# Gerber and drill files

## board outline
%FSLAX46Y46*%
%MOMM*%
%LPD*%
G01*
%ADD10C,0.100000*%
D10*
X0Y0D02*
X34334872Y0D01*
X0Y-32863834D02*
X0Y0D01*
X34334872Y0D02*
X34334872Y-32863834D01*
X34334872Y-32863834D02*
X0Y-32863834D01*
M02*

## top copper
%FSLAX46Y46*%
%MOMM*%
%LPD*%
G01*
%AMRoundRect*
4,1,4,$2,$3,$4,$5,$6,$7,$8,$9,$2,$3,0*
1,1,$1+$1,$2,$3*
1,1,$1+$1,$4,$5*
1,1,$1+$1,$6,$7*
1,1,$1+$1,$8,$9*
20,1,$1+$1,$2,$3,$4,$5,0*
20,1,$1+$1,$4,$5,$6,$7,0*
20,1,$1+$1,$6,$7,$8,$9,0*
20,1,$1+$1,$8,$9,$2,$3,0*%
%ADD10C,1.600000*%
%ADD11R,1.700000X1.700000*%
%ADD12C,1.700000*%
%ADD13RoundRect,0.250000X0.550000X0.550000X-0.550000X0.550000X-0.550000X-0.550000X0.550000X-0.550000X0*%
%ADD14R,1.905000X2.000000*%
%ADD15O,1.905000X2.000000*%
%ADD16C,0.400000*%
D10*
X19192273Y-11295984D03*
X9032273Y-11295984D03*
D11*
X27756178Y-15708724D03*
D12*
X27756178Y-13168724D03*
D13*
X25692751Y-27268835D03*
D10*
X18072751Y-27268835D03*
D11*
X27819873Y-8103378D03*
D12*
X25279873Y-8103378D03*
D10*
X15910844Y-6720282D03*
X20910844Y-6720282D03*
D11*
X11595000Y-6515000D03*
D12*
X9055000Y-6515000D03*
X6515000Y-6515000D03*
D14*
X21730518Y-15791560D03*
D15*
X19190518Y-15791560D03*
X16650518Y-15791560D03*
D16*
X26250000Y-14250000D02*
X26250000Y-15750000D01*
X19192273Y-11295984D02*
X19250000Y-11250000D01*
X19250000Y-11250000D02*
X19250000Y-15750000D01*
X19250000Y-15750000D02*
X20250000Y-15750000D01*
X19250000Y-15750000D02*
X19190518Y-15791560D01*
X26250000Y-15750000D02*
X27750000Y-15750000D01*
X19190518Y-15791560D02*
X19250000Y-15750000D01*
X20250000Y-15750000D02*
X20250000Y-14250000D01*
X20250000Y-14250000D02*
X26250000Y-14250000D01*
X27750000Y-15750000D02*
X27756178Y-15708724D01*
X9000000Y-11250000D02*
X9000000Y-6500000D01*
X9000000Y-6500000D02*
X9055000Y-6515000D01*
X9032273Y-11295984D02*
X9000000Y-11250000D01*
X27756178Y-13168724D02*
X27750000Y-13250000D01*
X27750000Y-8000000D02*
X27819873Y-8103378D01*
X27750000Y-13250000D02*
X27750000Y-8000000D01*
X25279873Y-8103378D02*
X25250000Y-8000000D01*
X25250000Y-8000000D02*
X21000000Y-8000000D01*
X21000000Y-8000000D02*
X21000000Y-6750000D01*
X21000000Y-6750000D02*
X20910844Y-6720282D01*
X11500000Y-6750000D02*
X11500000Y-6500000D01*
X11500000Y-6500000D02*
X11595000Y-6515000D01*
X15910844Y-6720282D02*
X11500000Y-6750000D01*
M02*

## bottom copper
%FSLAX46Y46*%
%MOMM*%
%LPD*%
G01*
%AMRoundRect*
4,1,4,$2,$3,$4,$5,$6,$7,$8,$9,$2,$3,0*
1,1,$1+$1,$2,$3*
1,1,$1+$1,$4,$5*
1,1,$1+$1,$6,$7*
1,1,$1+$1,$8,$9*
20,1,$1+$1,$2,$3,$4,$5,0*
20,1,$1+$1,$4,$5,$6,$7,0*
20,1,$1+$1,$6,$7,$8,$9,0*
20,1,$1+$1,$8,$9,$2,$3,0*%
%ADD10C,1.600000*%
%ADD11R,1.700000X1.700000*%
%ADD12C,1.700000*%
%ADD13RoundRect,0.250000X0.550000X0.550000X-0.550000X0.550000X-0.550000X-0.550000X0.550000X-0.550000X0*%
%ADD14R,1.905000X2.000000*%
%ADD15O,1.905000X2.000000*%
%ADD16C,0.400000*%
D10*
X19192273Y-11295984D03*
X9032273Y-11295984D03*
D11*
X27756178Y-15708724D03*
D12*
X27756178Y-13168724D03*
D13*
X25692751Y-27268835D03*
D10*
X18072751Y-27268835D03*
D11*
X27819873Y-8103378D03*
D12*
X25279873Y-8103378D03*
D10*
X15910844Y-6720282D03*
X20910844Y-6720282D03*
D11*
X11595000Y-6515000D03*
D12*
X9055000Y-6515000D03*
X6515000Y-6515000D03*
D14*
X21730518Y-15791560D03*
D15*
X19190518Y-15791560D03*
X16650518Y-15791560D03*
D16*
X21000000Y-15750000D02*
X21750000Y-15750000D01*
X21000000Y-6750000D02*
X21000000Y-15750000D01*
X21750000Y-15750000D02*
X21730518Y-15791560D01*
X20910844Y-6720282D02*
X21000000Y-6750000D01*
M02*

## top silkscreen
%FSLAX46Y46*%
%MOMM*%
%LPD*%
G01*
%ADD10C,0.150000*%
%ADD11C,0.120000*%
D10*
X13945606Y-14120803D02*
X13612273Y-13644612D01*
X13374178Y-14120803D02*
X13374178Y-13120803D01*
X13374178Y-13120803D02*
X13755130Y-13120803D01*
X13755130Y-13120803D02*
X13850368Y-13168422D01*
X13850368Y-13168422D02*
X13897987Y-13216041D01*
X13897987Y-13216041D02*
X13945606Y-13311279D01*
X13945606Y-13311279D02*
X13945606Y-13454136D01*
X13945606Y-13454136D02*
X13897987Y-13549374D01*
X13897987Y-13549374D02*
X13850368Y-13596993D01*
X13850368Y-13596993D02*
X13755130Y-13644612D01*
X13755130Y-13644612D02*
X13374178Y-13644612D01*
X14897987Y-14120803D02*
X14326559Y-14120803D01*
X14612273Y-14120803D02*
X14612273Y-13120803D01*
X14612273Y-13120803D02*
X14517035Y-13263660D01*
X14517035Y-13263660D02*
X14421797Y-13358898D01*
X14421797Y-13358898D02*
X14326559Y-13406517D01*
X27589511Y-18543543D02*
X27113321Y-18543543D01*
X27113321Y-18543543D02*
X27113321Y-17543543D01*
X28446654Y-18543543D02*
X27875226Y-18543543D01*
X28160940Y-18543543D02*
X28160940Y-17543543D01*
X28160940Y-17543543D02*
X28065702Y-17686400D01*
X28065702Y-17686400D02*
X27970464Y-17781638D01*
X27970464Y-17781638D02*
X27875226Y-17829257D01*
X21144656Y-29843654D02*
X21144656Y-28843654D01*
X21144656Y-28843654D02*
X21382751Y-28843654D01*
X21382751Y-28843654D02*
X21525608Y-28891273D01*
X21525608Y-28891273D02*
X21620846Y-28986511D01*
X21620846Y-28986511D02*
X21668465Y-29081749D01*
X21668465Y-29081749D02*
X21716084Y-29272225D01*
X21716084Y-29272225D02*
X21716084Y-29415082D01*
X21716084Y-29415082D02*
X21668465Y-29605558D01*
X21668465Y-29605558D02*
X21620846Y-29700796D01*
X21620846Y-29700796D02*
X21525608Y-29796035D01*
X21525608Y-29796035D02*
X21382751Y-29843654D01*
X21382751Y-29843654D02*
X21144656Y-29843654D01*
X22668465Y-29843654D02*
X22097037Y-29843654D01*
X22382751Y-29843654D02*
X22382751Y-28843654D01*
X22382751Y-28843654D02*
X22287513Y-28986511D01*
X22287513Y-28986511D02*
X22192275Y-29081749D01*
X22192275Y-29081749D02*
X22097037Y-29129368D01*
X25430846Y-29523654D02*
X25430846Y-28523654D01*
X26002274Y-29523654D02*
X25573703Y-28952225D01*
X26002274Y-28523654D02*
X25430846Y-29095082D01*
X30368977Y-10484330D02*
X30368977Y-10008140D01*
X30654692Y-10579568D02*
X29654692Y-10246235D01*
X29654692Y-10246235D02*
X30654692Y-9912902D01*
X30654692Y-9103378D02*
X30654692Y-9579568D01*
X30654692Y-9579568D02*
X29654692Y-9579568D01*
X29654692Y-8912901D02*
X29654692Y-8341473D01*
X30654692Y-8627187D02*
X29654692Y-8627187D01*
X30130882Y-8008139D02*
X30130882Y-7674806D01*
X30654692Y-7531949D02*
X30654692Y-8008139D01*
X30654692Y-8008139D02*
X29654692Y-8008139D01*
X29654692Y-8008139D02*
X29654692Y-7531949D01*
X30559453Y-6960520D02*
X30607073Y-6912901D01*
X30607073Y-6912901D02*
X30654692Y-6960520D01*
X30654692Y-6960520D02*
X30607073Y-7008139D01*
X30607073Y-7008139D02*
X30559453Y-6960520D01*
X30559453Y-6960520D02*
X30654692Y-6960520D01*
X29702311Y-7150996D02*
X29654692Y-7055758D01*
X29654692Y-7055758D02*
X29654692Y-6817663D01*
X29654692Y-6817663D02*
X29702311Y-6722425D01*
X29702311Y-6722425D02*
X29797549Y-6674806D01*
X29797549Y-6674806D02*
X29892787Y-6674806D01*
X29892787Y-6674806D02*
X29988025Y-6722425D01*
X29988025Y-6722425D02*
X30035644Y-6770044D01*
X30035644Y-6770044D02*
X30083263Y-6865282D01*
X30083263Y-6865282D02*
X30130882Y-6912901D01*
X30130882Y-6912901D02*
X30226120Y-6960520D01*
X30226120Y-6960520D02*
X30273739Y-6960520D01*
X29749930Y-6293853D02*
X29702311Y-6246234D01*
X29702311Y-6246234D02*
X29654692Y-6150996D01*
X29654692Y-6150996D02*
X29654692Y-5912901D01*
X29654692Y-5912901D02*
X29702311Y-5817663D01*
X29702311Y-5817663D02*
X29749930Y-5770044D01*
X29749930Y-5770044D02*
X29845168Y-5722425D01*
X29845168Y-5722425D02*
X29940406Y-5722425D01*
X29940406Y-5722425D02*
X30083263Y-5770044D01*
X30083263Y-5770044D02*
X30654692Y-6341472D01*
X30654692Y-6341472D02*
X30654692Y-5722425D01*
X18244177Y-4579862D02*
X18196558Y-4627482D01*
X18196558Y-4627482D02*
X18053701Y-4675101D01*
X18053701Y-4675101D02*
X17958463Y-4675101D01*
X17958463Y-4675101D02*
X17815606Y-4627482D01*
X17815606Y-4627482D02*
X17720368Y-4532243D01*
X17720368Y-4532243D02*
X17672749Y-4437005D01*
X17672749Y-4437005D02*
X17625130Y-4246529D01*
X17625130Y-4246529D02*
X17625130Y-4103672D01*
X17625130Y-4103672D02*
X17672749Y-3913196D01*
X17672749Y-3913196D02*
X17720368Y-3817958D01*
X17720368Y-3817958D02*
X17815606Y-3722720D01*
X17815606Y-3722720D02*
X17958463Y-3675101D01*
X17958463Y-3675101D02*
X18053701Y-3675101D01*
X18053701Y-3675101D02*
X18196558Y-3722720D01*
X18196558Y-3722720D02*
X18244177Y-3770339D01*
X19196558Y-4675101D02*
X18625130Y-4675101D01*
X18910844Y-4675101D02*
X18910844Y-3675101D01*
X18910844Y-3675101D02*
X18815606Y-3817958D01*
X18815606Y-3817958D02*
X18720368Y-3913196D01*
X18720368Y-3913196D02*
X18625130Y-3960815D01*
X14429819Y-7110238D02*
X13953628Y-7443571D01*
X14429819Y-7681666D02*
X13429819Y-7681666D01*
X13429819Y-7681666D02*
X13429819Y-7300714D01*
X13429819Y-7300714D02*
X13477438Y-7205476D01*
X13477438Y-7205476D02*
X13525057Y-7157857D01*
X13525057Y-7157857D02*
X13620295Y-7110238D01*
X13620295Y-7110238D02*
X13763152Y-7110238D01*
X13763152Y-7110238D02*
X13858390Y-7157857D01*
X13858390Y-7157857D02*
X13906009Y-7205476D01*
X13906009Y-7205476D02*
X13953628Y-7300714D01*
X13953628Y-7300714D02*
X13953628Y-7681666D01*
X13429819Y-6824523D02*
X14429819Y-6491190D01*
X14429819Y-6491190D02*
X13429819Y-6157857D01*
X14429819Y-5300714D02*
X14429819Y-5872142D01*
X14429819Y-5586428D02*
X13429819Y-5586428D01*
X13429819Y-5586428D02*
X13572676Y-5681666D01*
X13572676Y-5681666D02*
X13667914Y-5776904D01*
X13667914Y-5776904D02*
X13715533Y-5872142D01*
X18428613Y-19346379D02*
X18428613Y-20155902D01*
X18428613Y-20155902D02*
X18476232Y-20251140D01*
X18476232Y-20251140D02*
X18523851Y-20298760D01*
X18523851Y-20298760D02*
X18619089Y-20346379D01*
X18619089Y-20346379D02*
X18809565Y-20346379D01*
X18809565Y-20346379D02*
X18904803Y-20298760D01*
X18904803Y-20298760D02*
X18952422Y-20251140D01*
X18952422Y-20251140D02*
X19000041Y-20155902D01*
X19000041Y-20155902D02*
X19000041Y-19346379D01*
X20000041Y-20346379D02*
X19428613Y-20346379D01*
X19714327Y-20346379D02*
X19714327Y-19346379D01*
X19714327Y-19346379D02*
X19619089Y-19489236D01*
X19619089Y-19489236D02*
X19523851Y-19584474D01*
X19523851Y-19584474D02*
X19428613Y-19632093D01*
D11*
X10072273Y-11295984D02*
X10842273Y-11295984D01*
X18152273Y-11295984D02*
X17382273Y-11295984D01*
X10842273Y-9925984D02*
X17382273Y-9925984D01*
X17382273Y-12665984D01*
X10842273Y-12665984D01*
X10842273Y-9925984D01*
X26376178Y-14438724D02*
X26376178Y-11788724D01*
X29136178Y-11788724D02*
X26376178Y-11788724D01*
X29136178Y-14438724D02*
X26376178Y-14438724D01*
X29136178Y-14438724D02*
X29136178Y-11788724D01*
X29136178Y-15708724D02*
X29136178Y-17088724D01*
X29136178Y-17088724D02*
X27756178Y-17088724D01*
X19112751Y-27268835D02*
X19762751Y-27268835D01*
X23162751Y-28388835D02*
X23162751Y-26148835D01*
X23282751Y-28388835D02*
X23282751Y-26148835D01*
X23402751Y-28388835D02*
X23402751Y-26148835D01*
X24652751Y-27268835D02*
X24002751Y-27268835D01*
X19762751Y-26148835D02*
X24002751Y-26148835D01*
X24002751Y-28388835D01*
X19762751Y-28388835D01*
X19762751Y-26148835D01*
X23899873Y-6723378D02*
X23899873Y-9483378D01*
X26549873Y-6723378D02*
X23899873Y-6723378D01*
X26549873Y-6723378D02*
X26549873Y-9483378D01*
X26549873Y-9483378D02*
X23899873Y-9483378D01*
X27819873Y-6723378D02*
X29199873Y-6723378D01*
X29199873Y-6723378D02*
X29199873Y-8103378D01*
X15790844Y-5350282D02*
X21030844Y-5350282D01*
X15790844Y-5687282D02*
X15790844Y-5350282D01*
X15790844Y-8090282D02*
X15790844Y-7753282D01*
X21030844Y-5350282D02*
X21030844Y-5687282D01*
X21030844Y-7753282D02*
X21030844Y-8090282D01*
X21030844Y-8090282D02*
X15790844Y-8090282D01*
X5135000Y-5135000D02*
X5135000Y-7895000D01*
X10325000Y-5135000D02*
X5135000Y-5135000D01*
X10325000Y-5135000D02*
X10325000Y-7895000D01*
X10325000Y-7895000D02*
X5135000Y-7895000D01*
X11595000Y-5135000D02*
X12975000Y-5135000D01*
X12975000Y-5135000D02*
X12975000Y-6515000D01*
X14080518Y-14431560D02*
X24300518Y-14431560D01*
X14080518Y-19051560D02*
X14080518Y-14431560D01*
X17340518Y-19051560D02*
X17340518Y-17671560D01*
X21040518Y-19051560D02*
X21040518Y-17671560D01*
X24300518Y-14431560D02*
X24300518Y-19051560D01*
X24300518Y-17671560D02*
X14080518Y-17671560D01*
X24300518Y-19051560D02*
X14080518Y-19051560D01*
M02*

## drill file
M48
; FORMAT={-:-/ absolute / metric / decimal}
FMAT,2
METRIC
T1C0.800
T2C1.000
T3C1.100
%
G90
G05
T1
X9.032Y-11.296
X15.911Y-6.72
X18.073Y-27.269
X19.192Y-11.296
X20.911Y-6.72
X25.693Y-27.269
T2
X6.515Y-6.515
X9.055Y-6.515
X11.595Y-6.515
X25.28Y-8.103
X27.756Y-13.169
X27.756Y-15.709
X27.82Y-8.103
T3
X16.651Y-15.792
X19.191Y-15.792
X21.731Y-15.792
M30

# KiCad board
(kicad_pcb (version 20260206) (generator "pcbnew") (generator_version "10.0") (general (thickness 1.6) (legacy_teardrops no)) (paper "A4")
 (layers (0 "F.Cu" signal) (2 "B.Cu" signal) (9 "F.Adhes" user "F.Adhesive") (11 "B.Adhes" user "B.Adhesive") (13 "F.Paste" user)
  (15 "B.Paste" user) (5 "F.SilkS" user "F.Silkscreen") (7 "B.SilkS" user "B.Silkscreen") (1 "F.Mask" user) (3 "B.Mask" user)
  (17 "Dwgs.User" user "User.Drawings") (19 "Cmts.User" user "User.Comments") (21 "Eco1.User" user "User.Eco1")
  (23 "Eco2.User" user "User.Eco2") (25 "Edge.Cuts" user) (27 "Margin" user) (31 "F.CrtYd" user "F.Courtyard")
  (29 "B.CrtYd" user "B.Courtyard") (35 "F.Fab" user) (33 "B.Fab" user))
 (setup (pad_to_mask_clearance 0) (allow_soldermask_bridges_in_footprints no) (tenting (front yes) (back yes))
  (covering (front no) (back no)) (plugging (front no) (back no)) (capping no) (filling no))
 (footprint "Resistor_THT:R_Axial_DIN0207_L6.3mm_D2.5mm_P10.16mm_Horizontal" (layer "F.Cu") (at 19.192273 11.295984 180)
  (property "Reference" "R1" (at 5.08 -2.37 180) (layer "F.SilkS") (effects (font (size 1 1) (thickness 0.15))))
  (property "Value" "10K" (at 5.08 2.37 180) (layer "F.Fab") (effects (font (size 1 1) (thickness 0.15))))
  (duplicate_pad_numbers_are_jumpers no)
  (fp_line (start 9.12 0) (end 8.35 0) (stroke (width 0.12) (type solid)) (layer "F.SilkS"))
  (fp_line (start 1.04 0) (end 1.81 0) (stroke (width 0.12) (type solid)) (layer "F.SilkS"))
  (fp_rect (start 1.81 -1.37) (end 8.35 1.37) (stroke (width 0.12) (type solid)) (fill no) (layer "F.SilkS"))
  (pad "1" thru_hole circle (at 0 0 180) (size 1.6 1.6) (drill 0.8) (layers "*.Cu" "*.Mask") (remove_unused_layers no) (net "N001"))
  (pad "2" thru_hole circle (at 10.16 0 180) (size 1.6 1.6) (drill 0.8) (layers "*.Cu" "*.Mask") (remove_unused_layers no) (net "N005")))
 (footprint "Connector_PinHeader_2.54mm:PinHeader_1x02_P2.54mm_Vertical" (layer "F.Cu") (at 27.756178 15.708724 180)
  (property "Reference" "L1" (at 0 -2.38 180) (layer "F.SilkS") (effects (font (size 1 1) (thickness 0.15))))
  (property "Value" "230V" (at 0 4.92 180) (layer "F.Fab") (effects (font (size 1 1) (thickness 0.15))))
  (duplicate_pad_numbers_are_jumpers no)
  (fp_line (start 1.38 1.27) (end 1.38 3.92) (stroke (width 0.12) (type solid)) (layer "F.SilkS"))
  (fp_line (start -1.38 3.92) (end 1.38 3.92) (stroke (width 0.12) (type solid)) (layer "F.SilkS"))
  (fp_line (start -1.38 1.27) (end 1.38 1.27) (stroke (width 0.12) (type solid)) (layer "F.SilkS"))
  (fp_line (start -1.38 1.27) (end -1.38 3.92) (stroke (width 0.12) (type solid)) (layer "F.SilkS"))
  (fp_line (start -1.38 0) (end -1.38 -1.38) (stroke (width 0.12) (type solid)) (layer "F.SilkS"))
  (fp_line (start -1.38 -1.38) (end 0 -1.38) (stroke (width 0.12) (type solid)) (layer "F.SilkS"))
  (pad "1" thru_hole rect (at 0 0 180) (size 1.7 1.7) (drill 1) (layers "*.Cu" "*.Mask") (remove_unused_layers no) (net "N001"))
  (pad "2" thru_hole circle (at 0 2.54 180) (size 1.7 1.7) (drill 1) (layers "*.Cu" "*.Mask") (remove_unused_layers no) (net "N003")))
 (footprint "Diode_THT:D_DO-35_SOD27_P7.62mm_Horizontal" (layer "F.Cu") (at 25.692751 27.268835 180)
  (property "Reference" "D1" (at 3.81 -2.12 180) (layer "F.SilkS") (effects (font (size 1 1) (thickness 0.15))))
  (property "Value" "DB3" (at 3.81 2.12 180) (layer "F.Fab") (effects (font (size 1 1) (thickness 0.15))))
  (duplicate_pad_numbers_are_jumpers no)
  (fp_line (start 6.58 0) (end 5.93 0) (stroke (width 0.12) (type solid)) (layer "F.SilkS"))
  (fp_line (start 2.53 -1.12) (end 2.53 1.12) (stroke (width 0.12) (type solid)) (layer "F.SilkS"))
  (fp_line (start 2.41 -1.12) (end 2.41 1.12) (stroke (width 0.12) (type solid)) (layer "F.SilkS"))
  (fp_line (start 2.29 -1.12) (end 2.29 1.12) (stroke (width 0.12) (type solid)) (layer "F.SilkS"))
  (fp_line (start 1.04 0) (end 1.69 0) (stroke (width 0.12) (type solid)) (layer "F.SilkS"))
  (fp_rect (start 1.69 -1.12) (end 5.93 1.12) (stroke (width 0.12) (type solid)) (fill no) (layer "F.SilkS"))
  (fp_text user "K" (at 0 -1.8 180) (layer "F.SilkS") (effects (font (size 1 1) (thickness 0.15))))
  (pad "1" thru_hole roundrect (at 0 0 180) (size 1.6 1.6) (drill 0.8) (layers "*.Cu" "*.Mask") (remove_unused_layers no)
   (roundrect_rratio 0.15625))
  (pad "2" thru_hole circle (at 7.62 0 180) (size 1.6 1.6) (drill 0.8) (layers "*.Cu" "*.Mask") (remove_unused_layers no)))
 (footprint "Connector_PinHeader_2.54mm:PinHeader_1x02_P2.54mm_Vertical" (layer "F.Cu") (at 27.819873 8.103378 -90)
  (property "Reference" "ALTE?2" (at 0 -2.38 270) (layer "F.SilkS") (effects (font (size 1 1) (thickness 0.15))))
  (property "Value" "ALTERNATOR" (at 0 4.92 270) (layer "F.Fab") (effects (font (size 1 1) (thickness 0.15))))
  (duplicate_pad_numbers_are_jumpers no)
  (fp_line (start -1.38 3.92) (end 1.38 3.92) (stroke (width 0.12) (type solid)) (layer "F.SilkS"))
  (fp_line (start -1.38 1.27) (end -1.38 3.92) (stroke (width 0.12) (type solid)) (layer "F.SilkS"))
  (fp_line (start -1.38 1.27) (end 1.38 1.27) (stroke (width 0.12) (type solid)) (layer "F.SilkS"))
  (fp_line (start 1.38 1.27) (end 1.38 3.92) (stroke (width 0.12) (type solid)) (layer "F.SilkS"))
  (fp_line (start -1.38 0) (end -1.38 -1.38) (stroke (width 0.12) (type solid)) (layer "F.SilkS"))
  (fp_line (start -1.38 -1.38) (end 0 -1.38) (stroke (width 0.12) (type solid)) (layer "F.SilkS"))
  (pad "1" thru_hole rect (at 0 0 270) (size 1.7 1.7) (drill 1) (layers "*.Cu" "*.Mask") (remove_unused_layers no) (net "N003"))
  (pad "2" thru_hole circle (at 0 2.54 270) (size 1.7 1.7) (drill 1) (layers "*.Cu" "*.Mask") (remove_unused_layers no) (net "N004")))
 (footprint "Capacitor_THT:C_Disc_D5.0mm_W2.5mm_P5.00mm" (layer "F.Cu") (at 15.910844 6.720282)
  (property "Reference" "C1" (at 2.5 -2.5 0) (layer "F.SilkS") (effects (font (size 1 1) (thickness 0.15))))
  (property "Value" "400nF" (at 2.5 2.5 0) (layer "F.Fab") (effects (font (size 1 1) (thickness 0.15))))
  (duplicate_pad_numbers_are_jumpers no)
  (fp_line (start -0.12 -1.37) (end 5.12 -1.37) (stroke (width 0.12) (type solid)) (layer "F.SilkS"))
  (fp_line (start -0.12 -1.033) (end -0.12 -1.37) (stroke (width 0.12) (type solid)) (layer "F.SilkS"))
  (fp_line (start -0.12 1.37) (end -0.12 1.033) (stroke (width 0.12) (type solid)) (layer "F.SilkS"))
  (fp_line (start 5.12 -1.37) (end 5.12 -1.033) (stroke (width 0.12) (type solid)) (layer "F.SilkS"))
  (fp_line (start 5.12 1.033) (end 5.12 1.37) (stroke (width 0.12) (type solid)) (layer "F.SilkS"))
  (fp_line (start 5.12 1.37) (end -0.12 1.37) (stroke (width 0.12) (type solid)) (layer "F.SilkS"))
  (pad "1" thru_hole circle (at 0 0) (size 1.6 1.6) (drill 0.8) (layers "*.Cu" "*.Mask") (remove_unused_layers no) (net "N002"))
  (pad "2" thru_hole circle (at 5 0) (size 1.6 1.6) (drill 0.8) (layers "*.Cu" "*.Mask") (remove_unused_layers no) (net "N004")))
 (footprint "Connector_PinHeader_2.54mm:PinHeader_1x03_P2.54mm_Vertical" (layer "F.Cu") (at 11.595 6.515 -90)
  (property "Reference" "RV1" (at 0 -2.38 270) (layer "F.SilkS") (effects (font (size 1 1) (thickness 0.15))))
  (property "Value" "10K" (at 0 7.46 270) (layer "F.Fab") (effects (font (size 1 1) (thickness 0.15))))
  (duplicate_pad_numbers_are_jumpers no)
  (fp_line (start -1.38 6.46) (end 1.38 6.46) (stroke (width 0.12) (type solid)) (layer "F.SilkS"))
  (fp_line (start -1.38 1.27) (end -1.38 6.46) (stroke (width 0.12) (type solid)) (layer "F.SilkS"))
  (fp_line (start -1.38 1.27) (end 1.38 1.27) (stroke (width 0.12) (type solid)) (layer "F.SilkS"))
  (fp_line (start 1.38 1.27) (end 1.38 6.46) (stroke (width 0.12) (type solid)) (layer "F.SilkS"))
  (fp_line (start -1.38 0) (end -1.38 -1.38) (stroke (width 0.12) (type solid)) (layer "F.SilkS"))
  (fp_line (start -1.38 -1.38) (end 0 -1.38) (stroke (width 0.12) (type solid)) (layer "F.SilkS"))
  (pad "1" thru_hole rect (at 0 0 270) (size 1.7 1.7) (drill 1) (layers "*.Cu" "*.Mask") (remove_unused_layers no) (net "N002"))
  (pad "2" thru_hole circle (at 0 2.54 270) (size 1.7 1.7) (drill 1) (layers "*.Cu" "*.Mask") (remove_unused_layers no) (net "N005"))
  (pad "3" thru_hole circle (at 0 5.08 270) (size 1.7 1.7) (drill 1) (layers "*.Cu" "*.Mask") (remove_unused_layers no)))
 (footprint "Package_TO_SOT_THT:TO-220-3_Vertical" (layer "F.Cu") (at 21.730518 15.79156 180)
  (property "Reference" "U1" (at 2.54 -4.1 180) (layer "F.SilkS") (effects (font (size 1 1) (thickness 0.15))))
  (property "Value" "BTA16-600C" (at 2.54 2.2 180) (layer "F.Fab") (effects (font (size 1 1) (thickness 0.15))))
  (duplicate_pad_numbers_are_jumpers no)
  (fp_line (start 7.65 1.36) (end -2.57 1.36) (stroke (width 0.12) (type solid)) (layer "F.SilkS"))
  (fp_line (start 7.65 -3.26) (end 7.65 1.36) (stroke (width 0.12) (type solid)) (layer "F.SilkS"))
  (fp_line (start 4.39 -3.26) (end 4.39 -1.88) (stroke (width 0.12) (type solid)) (layer "F.SilkS"))
  (fp_line (start 0.69 -3.26) (end 0.69 -1.88) (stroke (width 0.12) (type solid)) (layer "F.SilkS"))
  (fp_line (start -2.57 1.36) (end -2.57 -3.26) (stroke (width 0.12) (type solid)) (layer "F.SilkS"))
  (fp_line (start -2.57 -1.88) (end 7.65 -1.88) (stroke (width 0.12) (type solid)) (layer "F.SilkS"))
  (fp_line (start -2.57 -3.26) (end 7.65 -3.26) (stroke (width 0.12) (type solid)) (layer "F.SilkS"))
  (pad "1" thru_hole rect (at 0 0 180) (size 1.905 2) (drill 1.1) (layers "*.Cu" "*.Mask") (remove_unused_layers no) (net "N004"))
  (pad "2" thru_hole oval (at 2.54 0 180) (size 1.905 2) (drill 1.1) (layers "*.Cu" "*.Mask") (remove_unused_layers no) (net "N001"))
  (pad "3" thru_hole oval (at 5.08 0 180) (size 1.905 2) (drill 1.1) (layers "*.Cu" "*.Mask") (remove_unused_layers no) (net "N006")))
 (gr_line (start 0 0) (end 34.334872 0) (stroke (width 0.1) (type default)) (layer "Edge.Cuts"))
 (gr_line (start 0 32.863834) (end 0 0) (stroke (width 0.1) (type default)) (layer "Edge.Cuts"))
 (gr_line (start 34.334872 0) (end 34.334872 32.863834) (stroke (width 0.1) (type default)) (layer "Edge.Cuts"))
 (gr_line (start 34.334872 32.863834) (end 0 32.863834) (stroke (width 0.1) (type default)) (layer "Edge.Cuts"))
 (segment (start 26.25 14.25) (end 26.25 15.75) (width 0.4) (layer "F.Cu") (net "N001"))
 (segment (start 19.192273 11.295984) (end 19.25 11.25) (width 0.4) (layer "F.Cu") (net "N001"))
 (segment (start 19.25 11.25) (end 19.25 15.75) (width 0.4) (layer "F.Cu") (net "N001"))
 (segment (start 19.25 15.75) (end 20.25 15.75) (width 0.4) (layer "F.Cu") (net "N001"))
 (segment (start 19.25 15.75) (end 19.190518 15.79156) (width 0.4) (layer "F.Cu") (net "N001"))
 (segment (start 26.25 15.75) (end 27.75 15.75) (width 0.4) (layer "F.Cu") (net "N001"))
 (segment (start 19.190518 15.79156) (end 19.25 15.75) (width 0.4) (layer "F.Cu") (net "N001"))
 (segment (start 20.25 15.75) (end 20.25 14.25) (width 0.4) (layer "F.Cu") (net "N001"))
 (segment (start 20.25 14.25) (end 26.25 14.25) (width 0.4) (layer "F.Cu") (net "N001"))
 (segment (start 27.75 15.75) (end 27.756178 15.708724) (width 0.4) (layer "F.Cu") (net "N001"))
 (segment (start 9 11.25) (end 9 6.5) (width 0.4) (layer "F.Cu") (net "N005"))
 (segment (start 9 6.5) (end 9.055 6.515) (width 0.4) (layer "F.Cu") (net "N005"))
 (segment (start 9.032273 11.295984) (end 9 11.25) (width 0.4) (layer "F.Cu") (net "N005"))
 (segment (start 27.756178 13.168724) (end 27.75 13.25) (width 0.4) (layer "F.Cu") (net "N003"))
 (segment (start 27.75 8) (end 27.819873 8.103378) (width 0.4) (layer "F.Cu") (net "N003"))
 (segment (start 27.75 13.25) (end 27.75 8) (width 0.4) (layer "F.Cu") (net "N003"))
 (segment (start 25.279873 8.103378) (end 25.25 8) (width 0.4) (layer "F.Cu") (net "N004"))
 (segment (start 25.25 8) (end 21 8) (width 0.4) (layer "F.Cu") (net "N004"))
 (segment (start 21 8) (end 21 6.75) (width 0.4) (layer "F.Cu") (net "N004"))
 (segment (start 21 6.75) (end 20.910844 6.720282) (width 0.4) (layer "F.Cu") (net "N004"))
 (segment (start 21 15.75) (end 21.75 15.75) (width 0.4) (layer "B.Cu") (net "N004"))
 (segment (start 21 6.75) (end 21 15.75) (width 0.4) (layer "B.Cu") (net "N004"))
 (segment (start 21.75 15.75) (end 21.730518 15.79156) (width 0.4) (layer "B.Cu") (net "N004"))
 (segment (start 20.910844 6.720282) (end 21 6.75) (width 0.4) (layer "B.Cu") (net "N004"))
 (segment (start 11.5 6.75) (end 11.5 6.5) (width 0.4) (layer "F.Cu") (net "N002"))
 (segment (start 11.5 6.5) (end 11.595 6.515) (width 0.4) (layer "F.Cu") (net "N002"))
 (segment (start 15.910844 6.720282) (end 11.5 6.75) (width 0.4) (layer "F.Cu") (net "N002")))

